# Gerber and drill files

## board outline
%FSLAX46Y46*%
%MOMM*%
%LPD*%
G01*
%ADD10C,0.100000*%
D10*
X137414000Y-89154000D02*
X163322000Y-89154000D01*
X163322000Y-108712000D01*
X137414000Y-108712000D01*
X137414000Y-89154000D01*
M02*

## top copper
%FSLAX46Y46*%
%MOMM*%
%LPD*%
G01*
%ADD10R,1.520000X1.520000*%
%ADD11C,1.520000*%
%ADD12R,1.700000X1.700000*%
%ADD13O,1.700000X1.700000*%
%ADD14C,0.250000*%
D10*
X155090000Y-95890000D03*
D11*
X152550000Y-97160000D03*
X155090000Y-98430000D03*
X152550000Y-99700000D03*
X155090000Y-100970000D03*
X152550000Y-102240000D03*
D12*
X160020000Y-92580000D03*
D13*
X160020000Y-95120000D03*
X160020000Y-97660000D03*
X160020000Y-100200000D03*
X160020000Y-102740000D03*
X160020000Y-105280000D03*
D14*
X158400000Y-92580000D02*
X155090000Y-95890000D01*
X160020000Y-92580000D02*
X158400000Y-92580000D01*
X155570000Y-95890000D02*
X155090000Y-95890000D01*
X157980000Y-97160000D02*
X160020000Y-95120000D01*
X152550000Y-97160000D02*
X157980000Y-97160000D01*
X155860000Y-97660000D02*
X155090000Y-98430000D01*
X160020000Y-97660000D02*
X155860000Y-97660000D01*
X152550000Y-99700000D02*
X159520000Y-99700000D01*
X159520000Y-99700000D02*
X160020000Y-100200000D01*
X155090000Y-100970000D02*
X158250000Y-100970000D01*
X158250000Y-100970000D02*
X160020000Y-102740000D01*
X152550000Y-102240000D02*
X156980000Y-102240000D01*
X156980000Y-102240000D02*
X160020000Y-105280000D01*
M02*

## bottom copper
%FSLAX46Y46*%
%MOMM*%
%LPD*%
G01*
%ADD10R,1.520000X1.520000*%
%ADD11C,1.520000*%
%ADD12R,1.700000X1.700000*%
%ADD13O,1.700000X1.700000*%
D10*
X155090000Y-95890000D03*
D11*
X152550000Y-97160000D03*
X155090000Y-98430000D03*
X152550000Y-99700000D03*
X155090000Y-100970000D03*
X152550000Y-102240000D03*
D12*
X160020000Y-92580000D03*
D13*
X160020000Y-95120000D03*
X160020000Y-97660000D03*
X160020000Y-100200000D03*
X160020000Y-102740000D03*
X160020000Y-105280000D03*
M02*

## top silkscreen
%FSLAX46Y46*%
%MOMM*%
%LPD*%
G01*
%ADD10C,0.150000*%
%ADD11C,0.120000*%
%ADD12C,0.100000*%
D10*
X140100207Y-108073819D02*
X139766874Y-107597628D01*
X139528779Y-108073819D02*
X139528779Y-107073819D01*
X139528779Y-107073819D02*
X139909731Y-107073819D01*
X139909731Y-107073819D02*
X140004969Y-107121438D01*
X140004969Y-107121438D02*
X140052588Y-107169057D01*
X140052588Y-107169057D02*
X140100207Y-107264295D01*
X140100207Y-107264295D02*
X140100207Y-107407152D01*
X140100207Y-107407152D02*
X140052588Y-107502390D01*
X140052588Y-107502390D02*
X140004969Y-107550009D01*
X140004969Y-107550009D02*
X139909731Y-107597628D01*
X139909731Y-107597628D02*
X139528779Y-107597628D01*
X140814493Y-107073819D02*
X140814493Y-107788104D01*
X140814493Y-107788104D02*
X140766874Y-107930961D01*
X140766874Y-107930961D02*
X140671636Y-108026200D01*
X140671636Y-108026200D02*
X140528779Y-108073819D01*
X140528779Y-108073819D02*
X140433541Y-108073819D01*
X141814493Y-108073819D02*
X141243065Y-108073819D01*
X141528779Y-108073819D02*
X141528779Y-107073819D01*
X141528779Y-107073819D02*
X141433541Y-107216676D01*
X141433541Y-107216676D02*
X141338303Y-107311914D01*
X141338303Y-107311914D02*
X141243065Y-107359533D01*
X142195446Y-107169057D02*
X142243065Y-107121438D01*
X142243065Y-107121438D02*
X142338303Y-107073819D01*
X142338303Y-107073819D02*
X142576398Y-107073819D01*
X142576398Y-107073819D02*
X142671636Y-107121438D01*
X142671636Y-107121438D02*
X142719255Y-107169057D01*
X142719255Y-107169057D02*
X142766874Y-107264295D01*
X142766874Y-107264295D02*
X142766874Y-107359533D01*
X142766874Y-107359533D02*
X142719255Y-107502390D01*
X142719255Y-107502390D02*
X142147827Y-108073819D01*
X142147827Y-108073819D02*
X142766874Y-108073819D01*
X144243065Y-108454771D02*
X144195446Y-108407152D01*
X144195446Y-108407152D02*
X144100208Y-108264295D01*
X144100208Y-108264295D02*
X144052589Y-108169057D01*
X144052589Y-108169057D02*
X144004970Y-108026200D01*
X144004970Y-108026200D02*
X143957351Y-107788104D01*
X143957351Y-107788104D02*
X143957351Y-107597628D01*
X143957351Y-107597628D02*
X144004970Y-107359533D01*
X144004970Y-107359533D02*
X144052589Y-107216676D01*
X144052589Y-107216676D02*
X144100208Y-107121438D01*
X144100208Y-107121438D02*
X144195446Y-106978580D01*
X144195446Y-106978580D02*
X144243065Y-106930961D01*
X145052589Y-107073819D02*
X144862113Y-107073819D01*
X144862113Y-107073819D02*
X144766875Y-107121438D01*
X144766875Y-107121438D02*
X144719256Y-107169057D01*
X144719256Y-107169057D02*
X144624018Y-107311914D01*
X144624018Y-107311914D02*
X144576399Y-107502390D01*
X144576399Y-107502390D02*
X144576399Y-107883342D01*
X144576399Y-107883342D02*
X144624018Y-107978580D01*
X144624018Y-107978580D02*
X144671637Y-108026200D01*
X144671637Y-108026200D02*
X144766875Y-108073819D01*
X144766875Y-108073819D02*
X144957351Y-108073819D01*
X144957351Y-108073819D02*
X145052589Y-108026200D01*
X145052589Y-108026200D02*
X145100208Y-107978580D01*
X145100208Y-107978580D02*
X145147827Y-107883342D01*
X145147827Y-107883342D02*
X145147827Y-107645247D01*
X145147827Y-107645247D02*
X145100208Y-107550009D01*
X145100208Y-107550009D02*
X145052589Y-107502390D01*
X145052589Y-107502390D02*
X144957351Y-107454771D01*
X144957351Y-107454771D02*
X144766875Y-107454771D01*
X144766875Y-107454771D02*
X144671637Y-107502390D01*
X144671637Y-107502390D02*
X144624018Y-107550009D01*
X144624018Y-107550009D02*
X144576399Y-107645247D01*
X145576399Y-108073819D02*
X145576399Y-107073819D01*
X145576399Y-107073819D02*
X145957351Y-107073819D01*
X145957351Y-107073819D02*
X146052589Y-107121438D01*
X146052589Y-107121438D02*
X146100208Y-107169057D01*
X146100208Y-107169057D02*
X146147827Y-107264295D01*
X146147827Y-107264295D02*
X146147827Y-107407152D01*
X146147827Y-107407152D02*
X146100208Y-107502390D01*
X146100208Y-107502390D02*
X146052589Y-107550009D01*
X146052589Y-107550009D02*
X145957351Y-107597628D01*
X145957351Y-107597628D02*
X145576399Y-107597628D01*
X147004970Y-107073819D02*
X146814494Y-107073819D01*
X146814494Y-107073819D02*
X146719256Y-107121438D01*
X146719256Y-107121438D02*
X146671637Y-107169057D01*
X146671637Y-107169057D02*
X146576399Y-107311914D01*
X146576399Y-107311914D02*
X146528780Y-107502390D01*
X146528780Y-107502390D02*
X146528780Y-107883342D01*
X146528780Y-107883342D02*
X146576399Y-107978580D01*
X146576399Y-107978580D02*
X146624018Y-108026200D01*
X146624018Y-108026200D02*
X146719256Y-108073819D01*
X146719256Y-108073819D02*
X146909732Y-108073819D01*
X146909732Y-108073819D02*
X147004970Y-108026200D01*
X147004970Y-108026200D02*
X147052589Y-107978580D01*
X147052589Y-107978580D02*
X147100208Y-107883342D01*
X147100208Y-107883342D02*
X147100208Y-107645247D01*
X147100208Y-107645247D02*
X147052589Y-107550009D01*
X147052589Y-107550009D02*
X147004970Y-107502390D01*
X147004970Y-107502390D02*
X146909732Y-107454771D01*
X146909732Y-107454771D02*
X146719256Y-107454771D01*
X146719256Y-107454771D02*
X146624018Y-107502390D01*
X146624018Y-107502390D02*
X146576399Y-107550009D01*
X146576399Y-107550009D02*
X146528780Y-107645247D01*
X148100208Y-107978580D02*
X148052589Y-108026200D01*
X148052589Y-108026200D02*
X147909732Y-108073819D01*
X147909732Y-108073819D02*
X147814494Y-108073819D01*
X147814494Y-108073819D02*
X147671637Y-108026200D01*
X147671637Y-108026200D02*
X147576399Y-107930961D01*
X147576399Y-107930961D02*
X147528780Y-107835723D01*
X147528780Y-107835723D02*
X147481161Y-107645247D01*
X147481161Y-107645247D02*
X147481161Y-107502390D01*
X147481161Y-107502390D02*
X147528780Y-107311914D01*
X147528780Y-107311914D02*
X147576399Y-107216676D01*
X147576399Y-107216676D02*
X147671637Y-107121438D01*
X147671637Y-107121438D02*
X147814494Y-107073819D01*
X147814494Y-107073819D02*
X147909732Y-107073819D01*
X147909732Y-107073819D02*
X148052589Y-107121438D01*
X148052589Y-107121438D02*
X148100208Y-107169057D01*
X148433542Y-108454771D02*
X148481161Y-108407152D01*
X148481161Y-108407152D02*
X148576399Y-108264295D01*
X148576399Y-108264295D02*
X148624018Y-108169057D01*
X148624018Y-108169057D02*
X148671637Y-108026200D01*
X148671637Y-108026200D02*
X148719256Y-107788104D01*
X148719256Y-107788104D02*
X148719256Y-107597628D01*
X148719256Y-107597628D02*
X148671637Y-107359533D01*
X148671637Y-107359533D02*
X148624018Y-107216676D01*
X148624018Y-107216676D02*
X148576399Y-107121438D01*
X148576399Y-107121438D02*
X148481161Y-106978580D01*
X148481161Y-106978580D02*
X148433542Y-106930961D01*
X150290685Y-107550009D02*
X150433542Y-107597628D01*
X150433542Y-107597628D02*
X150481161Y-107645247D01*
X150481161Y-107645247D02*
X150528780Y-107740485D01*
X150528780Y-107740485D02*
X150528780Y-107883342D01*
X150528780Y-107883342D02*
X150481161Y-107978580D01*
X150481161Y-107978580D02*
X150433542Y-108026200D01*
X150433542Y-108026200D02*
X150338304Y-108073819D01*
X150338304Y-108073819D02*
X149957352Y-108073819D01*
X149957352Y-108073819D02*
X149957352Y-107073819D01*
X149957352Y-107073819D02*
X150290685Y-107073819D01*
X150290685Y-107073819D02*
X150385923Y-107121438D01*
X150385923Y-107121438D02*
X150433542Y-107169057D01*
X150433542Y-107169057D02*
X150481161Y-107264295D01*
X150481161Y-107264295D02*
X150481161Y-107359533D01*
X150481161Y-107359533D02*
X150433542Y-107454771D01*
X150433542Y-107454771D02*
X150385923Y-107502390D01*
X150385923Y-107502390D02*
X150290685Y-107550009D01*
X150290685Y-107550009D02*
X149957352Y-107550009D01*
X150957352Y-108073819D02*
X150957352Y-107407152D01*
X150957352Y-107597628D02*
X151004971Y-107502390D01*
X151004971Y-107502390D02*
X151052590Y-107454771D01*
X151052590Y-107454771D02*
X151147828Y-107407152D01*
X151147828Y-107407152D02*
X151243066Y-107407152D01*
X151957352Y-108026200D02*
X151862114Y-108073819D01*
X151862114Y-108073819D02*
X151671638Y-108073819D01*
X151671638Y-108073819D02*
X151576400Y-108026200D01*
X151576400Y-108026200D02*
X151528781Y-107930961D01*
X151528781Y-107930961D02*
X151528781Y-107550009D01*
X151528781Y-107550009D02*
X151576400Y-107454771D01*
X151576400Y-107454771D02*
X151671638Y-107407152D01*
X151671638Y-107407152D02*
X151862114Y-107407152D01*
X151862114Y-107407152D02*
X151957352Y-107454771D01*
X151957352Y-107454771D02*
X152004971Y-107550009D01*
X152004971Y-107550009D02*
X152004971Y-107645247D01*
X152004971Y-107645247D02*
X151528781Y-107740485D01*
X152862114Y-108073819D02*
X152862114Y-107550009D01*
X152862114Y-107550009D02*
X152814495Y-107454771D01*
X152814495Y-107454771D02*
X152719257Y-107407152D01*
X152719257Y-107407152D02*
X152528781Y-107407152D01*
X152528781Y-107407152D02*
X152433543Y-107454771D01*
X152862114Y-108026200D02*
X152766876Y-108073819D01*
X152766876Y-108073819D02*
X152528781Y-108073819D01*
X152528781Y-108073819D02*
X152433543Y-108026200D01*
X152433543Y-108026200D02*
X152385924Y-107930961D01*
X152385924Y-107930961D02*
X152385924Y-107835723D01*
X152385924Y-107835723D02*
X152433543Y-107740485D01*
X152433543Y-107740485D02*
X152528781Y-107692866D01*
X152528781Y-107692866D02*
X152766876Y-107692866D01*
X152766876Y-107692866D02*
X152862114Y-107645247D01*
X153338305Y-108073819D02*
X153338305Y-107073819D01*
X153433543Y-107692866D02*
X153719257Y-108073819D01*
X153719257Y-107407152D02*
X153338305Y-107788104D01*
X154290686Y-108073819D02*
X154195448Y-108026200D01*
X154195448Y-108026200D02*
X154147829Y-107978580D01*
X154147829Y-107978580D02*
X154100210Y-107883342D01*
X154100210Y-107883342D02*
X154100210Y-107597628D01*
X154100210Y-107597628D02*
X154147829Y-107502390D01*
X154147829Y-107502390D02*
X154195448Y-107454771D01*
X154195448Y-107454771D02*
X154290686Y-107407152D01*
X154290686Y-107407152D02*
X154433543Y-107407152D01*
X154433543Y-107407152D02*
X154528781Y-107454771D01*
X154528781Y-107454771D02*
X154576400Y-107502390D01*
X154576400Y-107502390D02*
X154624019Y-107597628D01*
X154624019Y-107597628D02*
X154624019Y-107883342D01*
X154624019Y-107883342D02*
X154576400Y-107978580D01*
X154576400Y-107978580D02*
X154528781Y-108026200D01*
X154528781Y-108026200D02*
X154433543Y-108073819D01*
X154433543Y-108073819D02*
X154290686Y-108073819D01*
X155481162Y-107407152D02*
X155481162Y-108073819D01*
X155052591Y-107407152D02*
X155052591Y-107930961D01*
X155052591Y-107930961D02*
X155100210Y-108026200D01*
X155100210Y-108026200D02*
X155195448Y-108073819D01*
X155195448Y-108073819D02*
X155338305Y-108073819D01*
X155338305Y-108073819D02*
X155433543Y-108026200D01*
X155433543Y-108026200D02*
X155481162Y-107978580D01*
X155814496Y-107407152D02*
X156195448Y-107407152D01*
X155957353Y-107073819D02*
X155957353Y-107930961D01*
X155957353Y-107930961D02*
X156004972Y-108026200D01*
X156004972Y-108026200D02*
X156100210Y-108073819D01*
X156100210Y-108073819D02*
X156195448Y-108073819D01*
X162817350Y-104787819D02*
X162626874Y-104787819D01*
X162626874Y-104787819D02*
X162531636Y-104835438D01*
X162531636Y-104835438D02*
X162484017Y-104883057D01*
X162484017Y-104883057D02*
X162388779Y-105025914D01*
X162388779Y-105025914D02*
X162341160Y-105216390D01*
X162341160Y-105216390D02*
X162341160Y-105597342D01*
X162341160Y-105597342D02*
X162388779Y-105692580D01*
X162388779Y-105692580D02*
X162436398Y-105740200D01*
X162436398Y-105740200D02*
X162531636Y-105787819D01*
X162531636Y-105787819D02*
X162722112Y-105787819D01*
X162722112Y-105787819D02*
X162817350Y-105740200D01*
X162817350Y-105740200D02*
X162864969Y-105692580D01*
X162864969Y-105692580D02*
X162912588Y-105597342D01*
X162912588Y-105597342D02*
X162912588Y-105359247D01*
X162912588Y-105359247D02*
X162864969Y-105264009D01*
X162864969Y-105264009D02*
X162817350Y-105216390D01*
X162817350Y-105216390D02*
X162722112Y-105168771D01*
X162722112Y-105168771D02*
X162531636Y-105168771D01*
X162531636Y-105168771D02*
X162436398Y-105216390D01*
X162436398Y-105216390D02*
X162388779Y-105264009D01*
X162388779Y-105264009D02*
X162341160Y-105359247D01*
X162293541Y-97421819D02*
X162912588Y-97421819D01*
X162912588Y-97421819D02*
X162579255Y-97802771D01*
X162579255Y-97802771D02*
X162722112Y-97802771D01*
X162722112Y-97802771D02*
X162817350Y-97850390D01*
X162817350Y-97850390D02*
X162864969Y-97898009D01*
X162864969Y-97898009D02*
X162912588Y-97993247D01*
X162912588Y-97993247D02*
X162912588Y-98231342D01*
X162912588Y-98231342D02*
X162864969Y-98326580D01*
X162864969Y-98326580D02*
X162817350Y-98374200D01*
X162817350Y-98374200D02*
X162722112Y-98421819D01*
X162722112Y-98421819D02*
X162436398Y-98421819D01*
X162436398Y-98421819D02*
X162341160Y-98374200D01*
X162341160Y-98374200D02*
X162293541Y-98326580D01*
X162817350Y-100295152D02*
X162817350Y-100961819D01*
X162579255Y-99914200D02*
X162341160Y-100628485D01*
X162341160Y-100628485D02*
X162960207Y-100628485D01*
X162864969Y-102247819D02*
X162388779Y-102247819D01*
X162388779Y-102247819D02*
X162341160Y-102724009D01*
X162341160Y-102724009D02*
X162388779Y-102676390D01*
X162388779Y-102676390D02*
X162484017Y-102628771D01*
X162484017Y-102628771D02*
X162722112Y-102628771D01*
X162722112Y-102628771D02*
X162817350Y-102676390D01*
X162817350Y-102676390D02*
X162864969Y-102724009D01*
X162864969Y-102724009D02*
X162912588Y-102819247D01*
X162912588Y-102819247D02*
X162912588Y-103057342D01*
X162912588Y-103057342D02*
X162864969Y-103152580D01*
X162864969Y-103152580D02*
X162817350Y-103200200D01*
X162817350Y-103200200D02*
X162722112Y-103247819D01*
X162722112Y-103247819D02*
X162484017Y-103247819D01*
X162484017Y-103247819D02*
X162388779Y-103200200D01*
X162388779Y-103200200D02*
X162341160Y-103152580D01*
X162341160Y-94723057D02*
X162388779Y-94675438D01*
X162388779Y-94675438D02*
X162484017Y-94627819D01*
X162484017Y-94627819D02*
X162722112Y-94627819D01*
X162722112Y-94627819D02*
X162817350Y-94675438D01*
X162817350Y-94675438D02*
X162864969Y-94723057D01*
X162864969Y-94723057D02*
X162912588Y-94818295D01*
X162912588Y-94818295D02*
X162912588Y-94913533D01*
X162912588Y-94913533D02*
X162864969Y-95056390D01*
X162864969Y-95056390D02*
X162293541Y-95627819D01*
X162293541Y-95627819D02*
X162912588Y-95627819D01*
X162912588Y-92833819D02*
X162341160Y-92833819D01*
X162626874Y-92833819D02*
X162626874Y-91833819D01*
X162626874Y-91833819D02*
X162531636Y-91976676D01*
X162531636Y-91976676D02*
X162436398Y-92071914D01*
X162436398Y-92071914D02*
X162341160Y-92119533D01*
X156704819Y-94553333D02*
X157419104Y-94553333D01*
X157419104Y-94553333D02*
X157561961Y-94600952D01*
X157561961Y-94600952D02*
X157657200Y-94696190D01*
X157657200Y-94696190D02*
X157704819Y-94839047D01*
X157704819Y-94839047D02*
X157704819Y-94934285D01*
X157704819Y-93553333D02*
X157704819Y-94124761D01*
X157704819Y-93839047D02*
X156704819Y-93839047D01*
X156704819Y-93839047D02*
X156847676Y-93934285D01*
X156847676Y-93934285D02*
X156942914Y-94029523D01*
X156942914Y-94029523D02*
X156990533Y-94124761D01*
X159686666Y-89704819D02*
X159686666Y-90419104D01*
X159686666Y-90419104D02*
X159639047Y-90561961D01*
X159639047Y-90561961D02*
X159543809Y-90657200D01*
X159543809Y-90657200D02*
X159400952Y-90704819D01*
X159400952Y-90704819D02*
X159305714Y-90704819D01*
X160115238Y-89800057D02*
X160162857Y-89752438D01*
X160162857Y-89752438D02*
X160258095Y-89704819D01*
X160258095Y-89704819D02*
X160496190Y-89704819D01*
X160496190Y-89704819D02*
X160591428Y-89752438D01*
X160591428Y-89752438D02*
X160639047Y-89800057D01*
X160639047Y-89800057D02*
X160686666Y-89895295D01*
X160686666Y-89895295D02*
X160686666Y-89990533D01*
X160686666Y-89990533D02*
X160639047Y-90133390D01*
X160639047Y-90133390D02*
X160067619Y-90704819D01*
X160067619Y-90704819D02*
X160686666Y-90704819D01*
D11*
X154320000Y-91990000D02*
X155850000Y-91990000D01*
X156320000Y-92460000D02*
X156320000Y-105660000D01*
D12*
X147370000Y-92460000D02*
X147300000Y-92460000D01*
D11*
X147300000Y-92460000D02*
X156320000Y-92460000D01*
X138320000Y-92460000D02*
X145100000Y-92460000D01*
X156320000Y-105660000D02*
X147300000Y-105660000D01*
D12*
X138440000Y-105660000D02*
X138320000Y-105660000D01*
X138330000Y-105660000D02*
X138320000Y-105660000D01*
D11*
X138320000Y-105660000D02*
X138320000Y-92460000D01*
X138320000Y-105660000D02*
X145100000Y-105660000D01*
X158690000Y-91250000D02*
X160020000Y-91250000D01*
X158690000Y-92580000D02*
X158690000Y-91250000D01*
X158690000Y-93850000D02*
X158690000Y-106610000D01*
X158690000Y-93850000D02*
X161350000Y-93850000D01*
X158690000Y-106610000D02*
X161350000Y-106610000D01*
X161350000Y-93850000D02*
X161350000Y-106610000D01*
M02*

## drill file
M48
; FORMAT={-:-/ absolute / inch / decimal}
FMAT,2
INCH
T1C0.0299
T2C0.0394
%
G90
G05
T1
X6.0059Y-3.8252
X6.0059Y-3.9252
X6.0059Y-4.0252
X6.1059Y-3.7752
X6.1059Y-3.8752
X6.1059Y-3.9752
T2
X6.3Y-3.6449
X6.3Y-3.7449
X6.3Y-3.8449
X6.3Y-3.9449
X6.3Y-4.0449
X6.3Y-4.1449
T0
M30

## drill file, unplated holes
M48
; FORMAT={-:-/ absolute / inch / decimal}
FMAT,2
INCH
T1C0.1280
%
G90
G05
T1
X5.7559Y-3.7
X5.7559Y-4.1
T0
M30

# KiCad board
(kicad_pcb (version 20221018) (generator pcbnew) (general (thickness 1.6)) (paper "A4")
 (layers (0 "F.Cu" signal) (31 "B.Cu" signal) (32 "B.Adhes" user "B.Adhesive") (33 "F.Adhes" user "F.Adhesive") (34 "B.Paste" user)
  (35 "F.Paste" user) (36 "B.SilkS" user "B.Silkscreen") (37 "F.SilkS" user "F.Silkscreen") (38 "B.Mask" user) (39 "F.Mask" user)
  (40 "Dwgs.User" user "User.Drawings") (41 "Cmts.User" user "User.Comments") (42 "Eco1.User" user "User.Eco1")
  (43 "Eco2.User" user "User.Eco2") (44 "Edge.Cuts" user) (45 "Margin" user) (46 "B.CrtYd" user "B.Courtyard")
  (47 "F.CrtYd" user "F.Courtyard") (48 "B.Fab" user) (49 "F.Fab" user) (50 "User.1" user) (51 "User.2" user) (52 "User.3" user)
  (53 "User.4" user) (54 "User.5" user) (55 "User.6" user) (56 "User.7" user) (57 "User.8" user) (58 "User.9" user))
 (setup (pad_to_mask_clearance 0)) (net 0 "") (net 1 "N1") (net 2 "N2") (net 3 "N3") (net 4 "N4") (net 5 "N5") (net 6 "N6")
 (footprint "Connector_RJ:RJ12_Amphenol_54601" (layer "F.Cu") (at 155.09 95.89 -90)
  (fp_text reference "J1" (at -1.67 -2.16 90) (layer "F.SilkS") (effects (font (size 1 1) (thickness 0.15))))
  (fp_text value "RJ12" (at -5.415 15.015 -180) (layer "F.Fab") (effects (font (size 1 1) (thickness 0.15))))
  (fp_line (start -3.9 0.77) (end -3.9 -0.76) (stroke (width 0.12) (type solid)) (layer "F.SilkS"))
  (fp_line (start -3.43 -1.23) (end 9.77 -1.23) (stroke (width 0.12) (type solid)) (layer "F.SilkS"))
  (fp_line (start -3.43 7.72) (end -3.43 7.79) (stroke (width 0.1) (type solid)) (layer "F.SilkS"))
  (fp_line (start -3.43 7.79) (end -3.43 -1.23) (stroke (width 0.12) (type solid)) (layer "F.SilkS"))
  (fp_line (start -3.43 16.77) (end -3.43 9.99) (stroke (width 0.12) (type solid)) (layer "F.SilkS"))
  (fp_line (start 9.77 -1.23) (end 9.77 7.79) (stroke (width 0.12) (type solid)) (layer "F.SilkS"))
  (fp_line (start 9.77 16.65) (end 9.77 16.77) (stroke (width 0.1) (type solid)) (layer "F.SilkS"))
  (fp_line (start 9.77 16.76) (end 9.77 16.77) (stroke (width 0.1) (type solid)) (layer "F.SilkS"))
  (fp_line (start 9.77 16.77) (end -3.43 16.77) (stroke (width 0.12) (type solid)) (layer "F.SilkS"))
  (fp_line (start 9.77 16.77) (end 9.77 9.99) (stroke (width 0.12) (type solid)) (layer "F.SilkS"))
  (pad "" np_thru_hole circle (at -1.91 8.89 270) (size 3.25 3.25) (drill 3.25) (layers "*.Cu" "*.Mask"))
  (pad "" np_thru_hole circle (at 8.25 8.89 270) (size 3.25 3.25) (drill 3.25) (layers "*.Cu" "*.Mask"))
  (pad "1" thru_hole rect (at 0 0 270) (size 1.52 1.52) (drill 0.76) (layers "*.Cu" "*.Mask") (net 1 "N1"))
  (pad "2" thru_hole circle (at 1.27 2.54 270) (size 1.52 1.52) (drill 0.76) (layers "*.Cu" "*.Mask") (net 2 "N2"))
  (pad "3" thru_hole circle (at 2.54 0 270) (size 1.52 1.52) (drill 0.76) (layers "*.Cu" "*.Mask") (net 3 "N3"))
  (pad "4" thru_hole circle (at 3.81 2.54 270) (size 1.52 1.52) (drill 0.76) (layers "*.Cu" "*.Mask") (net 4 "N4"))
  (pad "5" thru_hole circle (at 5.08 0 270) (size 1.52 1.52) (drill 0.76) (layers "*.Cu" "*.Mask") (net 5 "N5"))
  (pad "6" thru_hole circle (at 6.35 2.54 270) (size 1.52 1.52) (drill 0.76) (layers "*.Cu" "*.Mask") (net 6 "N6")))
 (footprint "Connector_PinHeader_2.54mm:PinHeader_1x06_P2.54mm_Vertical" (layer "F.Cu") (at 160.02 92.58)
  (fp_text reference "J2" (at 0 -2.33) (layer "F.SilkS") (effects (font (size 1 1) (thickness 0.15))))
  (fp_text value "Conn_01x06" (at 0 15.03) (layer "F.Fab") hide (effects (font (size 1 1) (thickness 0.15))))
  (fp_line (start -1.33 -1.33) (end 0 -1.33) (stroke (width 0.12) (type solid)) (layer "F.SilkS"))
  (fp_line (start -1.33 0) (end -1.33 -1.33) (stroke (width 0.12) (type solid)) (layer "F.SilkS"))
  (fp_line (start -1.33 1.27) (end -1.33 14.03) (stroke (width 0.12) (type solid)) (layer "F.SilkS"))
  (fp_line (start -1.33 1.27) (end 1.33 1.27) (stroke (width 0.12) (type solid)) (layer "F.SilkS"))
  (fp_line (start -1.33 14.03) (end 1.33 14.03) (stroke (width 0.12) (type solid)) (layer "F.SilkS"))
  (fp_line (start 1.33 1.27) (end 1.33 14.03) (stroke (width 0.12) (type solid)) (layer "F.SilkS"))
  (pad "1" thru_hole rect (at 0 0) (size 1.7 1.7) (drill 1) (layers "*.Cu" "*.Mask") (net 1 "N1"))
  (pad "2" thru_hole oval (at 0 2.54) (size 1.7 1.7) (drill 1) (layers "*.Cu" "*.Mask") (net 2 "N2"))
  (pad "3" thru_hole oval (at 0 5.08) (size 1.7 1.7) (drill 1) (layers "*.Cu" "*.Mask") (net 3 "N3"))
  (pad "4" thru_hole oval (at 0 7.62) (size 1.7 1.7) (drill 1) (layers "*.Cu" "*.Mask") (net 4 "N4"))
  (pad "5" thru_hole oval (at 0 10.16) (size 1.7 1.7) (drill 1) (layers "*.Cu" "*.Mask") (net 5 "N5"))
  (pad "6" thru_hole oval (at 0 12.7) (size 1.7 1.7) (drill 1) (layers "*.Cu" "*.Mask") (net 6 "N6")))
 (gr_rect (start 137.414 89.154) (end 163.322 108.712) (stroke (width 0.1) (type default)) (fill none) (layer "Edge.Cuts"))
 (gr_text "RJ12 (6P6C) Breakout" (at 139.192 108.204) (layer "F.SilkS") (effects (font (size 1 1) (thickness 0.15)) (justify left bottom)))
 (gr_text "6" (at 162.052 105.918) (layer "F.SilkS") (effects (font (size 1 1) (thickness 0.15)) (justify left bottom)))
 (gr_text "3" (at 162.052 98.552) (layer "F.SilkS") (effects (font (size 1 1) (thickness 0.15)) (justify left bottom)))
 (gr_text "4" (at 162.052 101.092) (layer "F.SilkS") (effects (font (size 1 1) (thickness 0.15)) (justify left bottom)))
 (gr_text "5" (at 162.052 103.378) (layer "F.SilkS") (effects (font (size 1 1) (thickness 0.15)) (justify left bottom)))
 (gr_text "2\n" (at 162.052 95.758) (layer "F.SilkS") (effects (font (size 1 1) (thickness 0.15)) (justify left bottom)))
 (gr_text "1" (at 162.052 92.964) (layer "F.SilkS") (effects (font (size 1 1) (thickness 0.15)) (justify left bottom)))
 (segment (start 158.4 92.58) (end 155.09 95.89) (width 0.25) (layer "F.Cu") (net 1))
 (segment (start 160.02 92.58) (end 158.4 92.58) (width 0.25) (layer "F.Cu") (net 1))
 (segment (start 155.57 95.89) (end 155.09 95.89) (width 0.25) (layer "F.Cu") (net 1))
 (segment (start 157.98 97.16) (end 160.02 95.12) (width 0.25) (layer "F.Cu") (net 2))
 (segment (start 152.55 97.16) (end 157.98 97.16) (width 0.25) (layer "F.Cu") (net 2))
 (segment (start 155.86 97.66) (end 155.09 98.43) (width 0.25) (layer "F.Cu") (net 3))
 (segment (start 160.02 97.66) (end 155.86 97.66) (width 0.25) (layer "F.Cu") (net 3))
 (segment (start 152.55 99.7) (end 159.52 99.7) (width 0.25) (layer "F.Cu") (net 4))
 (segment (start 159.52 99.7) (end 160.02 100.2) (width 0.25) (layer "F.Cu") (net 4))
 (segment (start 155.09 100.97) (end 158.25 100.97) (width 0.25) (layer "F.Cu") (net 5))
 (segment (start 158.25 100.97) (end 160.02 102.74) (width 0.25) (layer "F.Cu") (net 5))
 (segment (start 152.55 102.24) (end 156.98 102.24) (width 0.25) (layer "F.Cu") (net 6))
 (segment (start 156.98 102.24) (end 160.02 105.28) (width 0.25) (layer "F.Cu") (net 6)))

